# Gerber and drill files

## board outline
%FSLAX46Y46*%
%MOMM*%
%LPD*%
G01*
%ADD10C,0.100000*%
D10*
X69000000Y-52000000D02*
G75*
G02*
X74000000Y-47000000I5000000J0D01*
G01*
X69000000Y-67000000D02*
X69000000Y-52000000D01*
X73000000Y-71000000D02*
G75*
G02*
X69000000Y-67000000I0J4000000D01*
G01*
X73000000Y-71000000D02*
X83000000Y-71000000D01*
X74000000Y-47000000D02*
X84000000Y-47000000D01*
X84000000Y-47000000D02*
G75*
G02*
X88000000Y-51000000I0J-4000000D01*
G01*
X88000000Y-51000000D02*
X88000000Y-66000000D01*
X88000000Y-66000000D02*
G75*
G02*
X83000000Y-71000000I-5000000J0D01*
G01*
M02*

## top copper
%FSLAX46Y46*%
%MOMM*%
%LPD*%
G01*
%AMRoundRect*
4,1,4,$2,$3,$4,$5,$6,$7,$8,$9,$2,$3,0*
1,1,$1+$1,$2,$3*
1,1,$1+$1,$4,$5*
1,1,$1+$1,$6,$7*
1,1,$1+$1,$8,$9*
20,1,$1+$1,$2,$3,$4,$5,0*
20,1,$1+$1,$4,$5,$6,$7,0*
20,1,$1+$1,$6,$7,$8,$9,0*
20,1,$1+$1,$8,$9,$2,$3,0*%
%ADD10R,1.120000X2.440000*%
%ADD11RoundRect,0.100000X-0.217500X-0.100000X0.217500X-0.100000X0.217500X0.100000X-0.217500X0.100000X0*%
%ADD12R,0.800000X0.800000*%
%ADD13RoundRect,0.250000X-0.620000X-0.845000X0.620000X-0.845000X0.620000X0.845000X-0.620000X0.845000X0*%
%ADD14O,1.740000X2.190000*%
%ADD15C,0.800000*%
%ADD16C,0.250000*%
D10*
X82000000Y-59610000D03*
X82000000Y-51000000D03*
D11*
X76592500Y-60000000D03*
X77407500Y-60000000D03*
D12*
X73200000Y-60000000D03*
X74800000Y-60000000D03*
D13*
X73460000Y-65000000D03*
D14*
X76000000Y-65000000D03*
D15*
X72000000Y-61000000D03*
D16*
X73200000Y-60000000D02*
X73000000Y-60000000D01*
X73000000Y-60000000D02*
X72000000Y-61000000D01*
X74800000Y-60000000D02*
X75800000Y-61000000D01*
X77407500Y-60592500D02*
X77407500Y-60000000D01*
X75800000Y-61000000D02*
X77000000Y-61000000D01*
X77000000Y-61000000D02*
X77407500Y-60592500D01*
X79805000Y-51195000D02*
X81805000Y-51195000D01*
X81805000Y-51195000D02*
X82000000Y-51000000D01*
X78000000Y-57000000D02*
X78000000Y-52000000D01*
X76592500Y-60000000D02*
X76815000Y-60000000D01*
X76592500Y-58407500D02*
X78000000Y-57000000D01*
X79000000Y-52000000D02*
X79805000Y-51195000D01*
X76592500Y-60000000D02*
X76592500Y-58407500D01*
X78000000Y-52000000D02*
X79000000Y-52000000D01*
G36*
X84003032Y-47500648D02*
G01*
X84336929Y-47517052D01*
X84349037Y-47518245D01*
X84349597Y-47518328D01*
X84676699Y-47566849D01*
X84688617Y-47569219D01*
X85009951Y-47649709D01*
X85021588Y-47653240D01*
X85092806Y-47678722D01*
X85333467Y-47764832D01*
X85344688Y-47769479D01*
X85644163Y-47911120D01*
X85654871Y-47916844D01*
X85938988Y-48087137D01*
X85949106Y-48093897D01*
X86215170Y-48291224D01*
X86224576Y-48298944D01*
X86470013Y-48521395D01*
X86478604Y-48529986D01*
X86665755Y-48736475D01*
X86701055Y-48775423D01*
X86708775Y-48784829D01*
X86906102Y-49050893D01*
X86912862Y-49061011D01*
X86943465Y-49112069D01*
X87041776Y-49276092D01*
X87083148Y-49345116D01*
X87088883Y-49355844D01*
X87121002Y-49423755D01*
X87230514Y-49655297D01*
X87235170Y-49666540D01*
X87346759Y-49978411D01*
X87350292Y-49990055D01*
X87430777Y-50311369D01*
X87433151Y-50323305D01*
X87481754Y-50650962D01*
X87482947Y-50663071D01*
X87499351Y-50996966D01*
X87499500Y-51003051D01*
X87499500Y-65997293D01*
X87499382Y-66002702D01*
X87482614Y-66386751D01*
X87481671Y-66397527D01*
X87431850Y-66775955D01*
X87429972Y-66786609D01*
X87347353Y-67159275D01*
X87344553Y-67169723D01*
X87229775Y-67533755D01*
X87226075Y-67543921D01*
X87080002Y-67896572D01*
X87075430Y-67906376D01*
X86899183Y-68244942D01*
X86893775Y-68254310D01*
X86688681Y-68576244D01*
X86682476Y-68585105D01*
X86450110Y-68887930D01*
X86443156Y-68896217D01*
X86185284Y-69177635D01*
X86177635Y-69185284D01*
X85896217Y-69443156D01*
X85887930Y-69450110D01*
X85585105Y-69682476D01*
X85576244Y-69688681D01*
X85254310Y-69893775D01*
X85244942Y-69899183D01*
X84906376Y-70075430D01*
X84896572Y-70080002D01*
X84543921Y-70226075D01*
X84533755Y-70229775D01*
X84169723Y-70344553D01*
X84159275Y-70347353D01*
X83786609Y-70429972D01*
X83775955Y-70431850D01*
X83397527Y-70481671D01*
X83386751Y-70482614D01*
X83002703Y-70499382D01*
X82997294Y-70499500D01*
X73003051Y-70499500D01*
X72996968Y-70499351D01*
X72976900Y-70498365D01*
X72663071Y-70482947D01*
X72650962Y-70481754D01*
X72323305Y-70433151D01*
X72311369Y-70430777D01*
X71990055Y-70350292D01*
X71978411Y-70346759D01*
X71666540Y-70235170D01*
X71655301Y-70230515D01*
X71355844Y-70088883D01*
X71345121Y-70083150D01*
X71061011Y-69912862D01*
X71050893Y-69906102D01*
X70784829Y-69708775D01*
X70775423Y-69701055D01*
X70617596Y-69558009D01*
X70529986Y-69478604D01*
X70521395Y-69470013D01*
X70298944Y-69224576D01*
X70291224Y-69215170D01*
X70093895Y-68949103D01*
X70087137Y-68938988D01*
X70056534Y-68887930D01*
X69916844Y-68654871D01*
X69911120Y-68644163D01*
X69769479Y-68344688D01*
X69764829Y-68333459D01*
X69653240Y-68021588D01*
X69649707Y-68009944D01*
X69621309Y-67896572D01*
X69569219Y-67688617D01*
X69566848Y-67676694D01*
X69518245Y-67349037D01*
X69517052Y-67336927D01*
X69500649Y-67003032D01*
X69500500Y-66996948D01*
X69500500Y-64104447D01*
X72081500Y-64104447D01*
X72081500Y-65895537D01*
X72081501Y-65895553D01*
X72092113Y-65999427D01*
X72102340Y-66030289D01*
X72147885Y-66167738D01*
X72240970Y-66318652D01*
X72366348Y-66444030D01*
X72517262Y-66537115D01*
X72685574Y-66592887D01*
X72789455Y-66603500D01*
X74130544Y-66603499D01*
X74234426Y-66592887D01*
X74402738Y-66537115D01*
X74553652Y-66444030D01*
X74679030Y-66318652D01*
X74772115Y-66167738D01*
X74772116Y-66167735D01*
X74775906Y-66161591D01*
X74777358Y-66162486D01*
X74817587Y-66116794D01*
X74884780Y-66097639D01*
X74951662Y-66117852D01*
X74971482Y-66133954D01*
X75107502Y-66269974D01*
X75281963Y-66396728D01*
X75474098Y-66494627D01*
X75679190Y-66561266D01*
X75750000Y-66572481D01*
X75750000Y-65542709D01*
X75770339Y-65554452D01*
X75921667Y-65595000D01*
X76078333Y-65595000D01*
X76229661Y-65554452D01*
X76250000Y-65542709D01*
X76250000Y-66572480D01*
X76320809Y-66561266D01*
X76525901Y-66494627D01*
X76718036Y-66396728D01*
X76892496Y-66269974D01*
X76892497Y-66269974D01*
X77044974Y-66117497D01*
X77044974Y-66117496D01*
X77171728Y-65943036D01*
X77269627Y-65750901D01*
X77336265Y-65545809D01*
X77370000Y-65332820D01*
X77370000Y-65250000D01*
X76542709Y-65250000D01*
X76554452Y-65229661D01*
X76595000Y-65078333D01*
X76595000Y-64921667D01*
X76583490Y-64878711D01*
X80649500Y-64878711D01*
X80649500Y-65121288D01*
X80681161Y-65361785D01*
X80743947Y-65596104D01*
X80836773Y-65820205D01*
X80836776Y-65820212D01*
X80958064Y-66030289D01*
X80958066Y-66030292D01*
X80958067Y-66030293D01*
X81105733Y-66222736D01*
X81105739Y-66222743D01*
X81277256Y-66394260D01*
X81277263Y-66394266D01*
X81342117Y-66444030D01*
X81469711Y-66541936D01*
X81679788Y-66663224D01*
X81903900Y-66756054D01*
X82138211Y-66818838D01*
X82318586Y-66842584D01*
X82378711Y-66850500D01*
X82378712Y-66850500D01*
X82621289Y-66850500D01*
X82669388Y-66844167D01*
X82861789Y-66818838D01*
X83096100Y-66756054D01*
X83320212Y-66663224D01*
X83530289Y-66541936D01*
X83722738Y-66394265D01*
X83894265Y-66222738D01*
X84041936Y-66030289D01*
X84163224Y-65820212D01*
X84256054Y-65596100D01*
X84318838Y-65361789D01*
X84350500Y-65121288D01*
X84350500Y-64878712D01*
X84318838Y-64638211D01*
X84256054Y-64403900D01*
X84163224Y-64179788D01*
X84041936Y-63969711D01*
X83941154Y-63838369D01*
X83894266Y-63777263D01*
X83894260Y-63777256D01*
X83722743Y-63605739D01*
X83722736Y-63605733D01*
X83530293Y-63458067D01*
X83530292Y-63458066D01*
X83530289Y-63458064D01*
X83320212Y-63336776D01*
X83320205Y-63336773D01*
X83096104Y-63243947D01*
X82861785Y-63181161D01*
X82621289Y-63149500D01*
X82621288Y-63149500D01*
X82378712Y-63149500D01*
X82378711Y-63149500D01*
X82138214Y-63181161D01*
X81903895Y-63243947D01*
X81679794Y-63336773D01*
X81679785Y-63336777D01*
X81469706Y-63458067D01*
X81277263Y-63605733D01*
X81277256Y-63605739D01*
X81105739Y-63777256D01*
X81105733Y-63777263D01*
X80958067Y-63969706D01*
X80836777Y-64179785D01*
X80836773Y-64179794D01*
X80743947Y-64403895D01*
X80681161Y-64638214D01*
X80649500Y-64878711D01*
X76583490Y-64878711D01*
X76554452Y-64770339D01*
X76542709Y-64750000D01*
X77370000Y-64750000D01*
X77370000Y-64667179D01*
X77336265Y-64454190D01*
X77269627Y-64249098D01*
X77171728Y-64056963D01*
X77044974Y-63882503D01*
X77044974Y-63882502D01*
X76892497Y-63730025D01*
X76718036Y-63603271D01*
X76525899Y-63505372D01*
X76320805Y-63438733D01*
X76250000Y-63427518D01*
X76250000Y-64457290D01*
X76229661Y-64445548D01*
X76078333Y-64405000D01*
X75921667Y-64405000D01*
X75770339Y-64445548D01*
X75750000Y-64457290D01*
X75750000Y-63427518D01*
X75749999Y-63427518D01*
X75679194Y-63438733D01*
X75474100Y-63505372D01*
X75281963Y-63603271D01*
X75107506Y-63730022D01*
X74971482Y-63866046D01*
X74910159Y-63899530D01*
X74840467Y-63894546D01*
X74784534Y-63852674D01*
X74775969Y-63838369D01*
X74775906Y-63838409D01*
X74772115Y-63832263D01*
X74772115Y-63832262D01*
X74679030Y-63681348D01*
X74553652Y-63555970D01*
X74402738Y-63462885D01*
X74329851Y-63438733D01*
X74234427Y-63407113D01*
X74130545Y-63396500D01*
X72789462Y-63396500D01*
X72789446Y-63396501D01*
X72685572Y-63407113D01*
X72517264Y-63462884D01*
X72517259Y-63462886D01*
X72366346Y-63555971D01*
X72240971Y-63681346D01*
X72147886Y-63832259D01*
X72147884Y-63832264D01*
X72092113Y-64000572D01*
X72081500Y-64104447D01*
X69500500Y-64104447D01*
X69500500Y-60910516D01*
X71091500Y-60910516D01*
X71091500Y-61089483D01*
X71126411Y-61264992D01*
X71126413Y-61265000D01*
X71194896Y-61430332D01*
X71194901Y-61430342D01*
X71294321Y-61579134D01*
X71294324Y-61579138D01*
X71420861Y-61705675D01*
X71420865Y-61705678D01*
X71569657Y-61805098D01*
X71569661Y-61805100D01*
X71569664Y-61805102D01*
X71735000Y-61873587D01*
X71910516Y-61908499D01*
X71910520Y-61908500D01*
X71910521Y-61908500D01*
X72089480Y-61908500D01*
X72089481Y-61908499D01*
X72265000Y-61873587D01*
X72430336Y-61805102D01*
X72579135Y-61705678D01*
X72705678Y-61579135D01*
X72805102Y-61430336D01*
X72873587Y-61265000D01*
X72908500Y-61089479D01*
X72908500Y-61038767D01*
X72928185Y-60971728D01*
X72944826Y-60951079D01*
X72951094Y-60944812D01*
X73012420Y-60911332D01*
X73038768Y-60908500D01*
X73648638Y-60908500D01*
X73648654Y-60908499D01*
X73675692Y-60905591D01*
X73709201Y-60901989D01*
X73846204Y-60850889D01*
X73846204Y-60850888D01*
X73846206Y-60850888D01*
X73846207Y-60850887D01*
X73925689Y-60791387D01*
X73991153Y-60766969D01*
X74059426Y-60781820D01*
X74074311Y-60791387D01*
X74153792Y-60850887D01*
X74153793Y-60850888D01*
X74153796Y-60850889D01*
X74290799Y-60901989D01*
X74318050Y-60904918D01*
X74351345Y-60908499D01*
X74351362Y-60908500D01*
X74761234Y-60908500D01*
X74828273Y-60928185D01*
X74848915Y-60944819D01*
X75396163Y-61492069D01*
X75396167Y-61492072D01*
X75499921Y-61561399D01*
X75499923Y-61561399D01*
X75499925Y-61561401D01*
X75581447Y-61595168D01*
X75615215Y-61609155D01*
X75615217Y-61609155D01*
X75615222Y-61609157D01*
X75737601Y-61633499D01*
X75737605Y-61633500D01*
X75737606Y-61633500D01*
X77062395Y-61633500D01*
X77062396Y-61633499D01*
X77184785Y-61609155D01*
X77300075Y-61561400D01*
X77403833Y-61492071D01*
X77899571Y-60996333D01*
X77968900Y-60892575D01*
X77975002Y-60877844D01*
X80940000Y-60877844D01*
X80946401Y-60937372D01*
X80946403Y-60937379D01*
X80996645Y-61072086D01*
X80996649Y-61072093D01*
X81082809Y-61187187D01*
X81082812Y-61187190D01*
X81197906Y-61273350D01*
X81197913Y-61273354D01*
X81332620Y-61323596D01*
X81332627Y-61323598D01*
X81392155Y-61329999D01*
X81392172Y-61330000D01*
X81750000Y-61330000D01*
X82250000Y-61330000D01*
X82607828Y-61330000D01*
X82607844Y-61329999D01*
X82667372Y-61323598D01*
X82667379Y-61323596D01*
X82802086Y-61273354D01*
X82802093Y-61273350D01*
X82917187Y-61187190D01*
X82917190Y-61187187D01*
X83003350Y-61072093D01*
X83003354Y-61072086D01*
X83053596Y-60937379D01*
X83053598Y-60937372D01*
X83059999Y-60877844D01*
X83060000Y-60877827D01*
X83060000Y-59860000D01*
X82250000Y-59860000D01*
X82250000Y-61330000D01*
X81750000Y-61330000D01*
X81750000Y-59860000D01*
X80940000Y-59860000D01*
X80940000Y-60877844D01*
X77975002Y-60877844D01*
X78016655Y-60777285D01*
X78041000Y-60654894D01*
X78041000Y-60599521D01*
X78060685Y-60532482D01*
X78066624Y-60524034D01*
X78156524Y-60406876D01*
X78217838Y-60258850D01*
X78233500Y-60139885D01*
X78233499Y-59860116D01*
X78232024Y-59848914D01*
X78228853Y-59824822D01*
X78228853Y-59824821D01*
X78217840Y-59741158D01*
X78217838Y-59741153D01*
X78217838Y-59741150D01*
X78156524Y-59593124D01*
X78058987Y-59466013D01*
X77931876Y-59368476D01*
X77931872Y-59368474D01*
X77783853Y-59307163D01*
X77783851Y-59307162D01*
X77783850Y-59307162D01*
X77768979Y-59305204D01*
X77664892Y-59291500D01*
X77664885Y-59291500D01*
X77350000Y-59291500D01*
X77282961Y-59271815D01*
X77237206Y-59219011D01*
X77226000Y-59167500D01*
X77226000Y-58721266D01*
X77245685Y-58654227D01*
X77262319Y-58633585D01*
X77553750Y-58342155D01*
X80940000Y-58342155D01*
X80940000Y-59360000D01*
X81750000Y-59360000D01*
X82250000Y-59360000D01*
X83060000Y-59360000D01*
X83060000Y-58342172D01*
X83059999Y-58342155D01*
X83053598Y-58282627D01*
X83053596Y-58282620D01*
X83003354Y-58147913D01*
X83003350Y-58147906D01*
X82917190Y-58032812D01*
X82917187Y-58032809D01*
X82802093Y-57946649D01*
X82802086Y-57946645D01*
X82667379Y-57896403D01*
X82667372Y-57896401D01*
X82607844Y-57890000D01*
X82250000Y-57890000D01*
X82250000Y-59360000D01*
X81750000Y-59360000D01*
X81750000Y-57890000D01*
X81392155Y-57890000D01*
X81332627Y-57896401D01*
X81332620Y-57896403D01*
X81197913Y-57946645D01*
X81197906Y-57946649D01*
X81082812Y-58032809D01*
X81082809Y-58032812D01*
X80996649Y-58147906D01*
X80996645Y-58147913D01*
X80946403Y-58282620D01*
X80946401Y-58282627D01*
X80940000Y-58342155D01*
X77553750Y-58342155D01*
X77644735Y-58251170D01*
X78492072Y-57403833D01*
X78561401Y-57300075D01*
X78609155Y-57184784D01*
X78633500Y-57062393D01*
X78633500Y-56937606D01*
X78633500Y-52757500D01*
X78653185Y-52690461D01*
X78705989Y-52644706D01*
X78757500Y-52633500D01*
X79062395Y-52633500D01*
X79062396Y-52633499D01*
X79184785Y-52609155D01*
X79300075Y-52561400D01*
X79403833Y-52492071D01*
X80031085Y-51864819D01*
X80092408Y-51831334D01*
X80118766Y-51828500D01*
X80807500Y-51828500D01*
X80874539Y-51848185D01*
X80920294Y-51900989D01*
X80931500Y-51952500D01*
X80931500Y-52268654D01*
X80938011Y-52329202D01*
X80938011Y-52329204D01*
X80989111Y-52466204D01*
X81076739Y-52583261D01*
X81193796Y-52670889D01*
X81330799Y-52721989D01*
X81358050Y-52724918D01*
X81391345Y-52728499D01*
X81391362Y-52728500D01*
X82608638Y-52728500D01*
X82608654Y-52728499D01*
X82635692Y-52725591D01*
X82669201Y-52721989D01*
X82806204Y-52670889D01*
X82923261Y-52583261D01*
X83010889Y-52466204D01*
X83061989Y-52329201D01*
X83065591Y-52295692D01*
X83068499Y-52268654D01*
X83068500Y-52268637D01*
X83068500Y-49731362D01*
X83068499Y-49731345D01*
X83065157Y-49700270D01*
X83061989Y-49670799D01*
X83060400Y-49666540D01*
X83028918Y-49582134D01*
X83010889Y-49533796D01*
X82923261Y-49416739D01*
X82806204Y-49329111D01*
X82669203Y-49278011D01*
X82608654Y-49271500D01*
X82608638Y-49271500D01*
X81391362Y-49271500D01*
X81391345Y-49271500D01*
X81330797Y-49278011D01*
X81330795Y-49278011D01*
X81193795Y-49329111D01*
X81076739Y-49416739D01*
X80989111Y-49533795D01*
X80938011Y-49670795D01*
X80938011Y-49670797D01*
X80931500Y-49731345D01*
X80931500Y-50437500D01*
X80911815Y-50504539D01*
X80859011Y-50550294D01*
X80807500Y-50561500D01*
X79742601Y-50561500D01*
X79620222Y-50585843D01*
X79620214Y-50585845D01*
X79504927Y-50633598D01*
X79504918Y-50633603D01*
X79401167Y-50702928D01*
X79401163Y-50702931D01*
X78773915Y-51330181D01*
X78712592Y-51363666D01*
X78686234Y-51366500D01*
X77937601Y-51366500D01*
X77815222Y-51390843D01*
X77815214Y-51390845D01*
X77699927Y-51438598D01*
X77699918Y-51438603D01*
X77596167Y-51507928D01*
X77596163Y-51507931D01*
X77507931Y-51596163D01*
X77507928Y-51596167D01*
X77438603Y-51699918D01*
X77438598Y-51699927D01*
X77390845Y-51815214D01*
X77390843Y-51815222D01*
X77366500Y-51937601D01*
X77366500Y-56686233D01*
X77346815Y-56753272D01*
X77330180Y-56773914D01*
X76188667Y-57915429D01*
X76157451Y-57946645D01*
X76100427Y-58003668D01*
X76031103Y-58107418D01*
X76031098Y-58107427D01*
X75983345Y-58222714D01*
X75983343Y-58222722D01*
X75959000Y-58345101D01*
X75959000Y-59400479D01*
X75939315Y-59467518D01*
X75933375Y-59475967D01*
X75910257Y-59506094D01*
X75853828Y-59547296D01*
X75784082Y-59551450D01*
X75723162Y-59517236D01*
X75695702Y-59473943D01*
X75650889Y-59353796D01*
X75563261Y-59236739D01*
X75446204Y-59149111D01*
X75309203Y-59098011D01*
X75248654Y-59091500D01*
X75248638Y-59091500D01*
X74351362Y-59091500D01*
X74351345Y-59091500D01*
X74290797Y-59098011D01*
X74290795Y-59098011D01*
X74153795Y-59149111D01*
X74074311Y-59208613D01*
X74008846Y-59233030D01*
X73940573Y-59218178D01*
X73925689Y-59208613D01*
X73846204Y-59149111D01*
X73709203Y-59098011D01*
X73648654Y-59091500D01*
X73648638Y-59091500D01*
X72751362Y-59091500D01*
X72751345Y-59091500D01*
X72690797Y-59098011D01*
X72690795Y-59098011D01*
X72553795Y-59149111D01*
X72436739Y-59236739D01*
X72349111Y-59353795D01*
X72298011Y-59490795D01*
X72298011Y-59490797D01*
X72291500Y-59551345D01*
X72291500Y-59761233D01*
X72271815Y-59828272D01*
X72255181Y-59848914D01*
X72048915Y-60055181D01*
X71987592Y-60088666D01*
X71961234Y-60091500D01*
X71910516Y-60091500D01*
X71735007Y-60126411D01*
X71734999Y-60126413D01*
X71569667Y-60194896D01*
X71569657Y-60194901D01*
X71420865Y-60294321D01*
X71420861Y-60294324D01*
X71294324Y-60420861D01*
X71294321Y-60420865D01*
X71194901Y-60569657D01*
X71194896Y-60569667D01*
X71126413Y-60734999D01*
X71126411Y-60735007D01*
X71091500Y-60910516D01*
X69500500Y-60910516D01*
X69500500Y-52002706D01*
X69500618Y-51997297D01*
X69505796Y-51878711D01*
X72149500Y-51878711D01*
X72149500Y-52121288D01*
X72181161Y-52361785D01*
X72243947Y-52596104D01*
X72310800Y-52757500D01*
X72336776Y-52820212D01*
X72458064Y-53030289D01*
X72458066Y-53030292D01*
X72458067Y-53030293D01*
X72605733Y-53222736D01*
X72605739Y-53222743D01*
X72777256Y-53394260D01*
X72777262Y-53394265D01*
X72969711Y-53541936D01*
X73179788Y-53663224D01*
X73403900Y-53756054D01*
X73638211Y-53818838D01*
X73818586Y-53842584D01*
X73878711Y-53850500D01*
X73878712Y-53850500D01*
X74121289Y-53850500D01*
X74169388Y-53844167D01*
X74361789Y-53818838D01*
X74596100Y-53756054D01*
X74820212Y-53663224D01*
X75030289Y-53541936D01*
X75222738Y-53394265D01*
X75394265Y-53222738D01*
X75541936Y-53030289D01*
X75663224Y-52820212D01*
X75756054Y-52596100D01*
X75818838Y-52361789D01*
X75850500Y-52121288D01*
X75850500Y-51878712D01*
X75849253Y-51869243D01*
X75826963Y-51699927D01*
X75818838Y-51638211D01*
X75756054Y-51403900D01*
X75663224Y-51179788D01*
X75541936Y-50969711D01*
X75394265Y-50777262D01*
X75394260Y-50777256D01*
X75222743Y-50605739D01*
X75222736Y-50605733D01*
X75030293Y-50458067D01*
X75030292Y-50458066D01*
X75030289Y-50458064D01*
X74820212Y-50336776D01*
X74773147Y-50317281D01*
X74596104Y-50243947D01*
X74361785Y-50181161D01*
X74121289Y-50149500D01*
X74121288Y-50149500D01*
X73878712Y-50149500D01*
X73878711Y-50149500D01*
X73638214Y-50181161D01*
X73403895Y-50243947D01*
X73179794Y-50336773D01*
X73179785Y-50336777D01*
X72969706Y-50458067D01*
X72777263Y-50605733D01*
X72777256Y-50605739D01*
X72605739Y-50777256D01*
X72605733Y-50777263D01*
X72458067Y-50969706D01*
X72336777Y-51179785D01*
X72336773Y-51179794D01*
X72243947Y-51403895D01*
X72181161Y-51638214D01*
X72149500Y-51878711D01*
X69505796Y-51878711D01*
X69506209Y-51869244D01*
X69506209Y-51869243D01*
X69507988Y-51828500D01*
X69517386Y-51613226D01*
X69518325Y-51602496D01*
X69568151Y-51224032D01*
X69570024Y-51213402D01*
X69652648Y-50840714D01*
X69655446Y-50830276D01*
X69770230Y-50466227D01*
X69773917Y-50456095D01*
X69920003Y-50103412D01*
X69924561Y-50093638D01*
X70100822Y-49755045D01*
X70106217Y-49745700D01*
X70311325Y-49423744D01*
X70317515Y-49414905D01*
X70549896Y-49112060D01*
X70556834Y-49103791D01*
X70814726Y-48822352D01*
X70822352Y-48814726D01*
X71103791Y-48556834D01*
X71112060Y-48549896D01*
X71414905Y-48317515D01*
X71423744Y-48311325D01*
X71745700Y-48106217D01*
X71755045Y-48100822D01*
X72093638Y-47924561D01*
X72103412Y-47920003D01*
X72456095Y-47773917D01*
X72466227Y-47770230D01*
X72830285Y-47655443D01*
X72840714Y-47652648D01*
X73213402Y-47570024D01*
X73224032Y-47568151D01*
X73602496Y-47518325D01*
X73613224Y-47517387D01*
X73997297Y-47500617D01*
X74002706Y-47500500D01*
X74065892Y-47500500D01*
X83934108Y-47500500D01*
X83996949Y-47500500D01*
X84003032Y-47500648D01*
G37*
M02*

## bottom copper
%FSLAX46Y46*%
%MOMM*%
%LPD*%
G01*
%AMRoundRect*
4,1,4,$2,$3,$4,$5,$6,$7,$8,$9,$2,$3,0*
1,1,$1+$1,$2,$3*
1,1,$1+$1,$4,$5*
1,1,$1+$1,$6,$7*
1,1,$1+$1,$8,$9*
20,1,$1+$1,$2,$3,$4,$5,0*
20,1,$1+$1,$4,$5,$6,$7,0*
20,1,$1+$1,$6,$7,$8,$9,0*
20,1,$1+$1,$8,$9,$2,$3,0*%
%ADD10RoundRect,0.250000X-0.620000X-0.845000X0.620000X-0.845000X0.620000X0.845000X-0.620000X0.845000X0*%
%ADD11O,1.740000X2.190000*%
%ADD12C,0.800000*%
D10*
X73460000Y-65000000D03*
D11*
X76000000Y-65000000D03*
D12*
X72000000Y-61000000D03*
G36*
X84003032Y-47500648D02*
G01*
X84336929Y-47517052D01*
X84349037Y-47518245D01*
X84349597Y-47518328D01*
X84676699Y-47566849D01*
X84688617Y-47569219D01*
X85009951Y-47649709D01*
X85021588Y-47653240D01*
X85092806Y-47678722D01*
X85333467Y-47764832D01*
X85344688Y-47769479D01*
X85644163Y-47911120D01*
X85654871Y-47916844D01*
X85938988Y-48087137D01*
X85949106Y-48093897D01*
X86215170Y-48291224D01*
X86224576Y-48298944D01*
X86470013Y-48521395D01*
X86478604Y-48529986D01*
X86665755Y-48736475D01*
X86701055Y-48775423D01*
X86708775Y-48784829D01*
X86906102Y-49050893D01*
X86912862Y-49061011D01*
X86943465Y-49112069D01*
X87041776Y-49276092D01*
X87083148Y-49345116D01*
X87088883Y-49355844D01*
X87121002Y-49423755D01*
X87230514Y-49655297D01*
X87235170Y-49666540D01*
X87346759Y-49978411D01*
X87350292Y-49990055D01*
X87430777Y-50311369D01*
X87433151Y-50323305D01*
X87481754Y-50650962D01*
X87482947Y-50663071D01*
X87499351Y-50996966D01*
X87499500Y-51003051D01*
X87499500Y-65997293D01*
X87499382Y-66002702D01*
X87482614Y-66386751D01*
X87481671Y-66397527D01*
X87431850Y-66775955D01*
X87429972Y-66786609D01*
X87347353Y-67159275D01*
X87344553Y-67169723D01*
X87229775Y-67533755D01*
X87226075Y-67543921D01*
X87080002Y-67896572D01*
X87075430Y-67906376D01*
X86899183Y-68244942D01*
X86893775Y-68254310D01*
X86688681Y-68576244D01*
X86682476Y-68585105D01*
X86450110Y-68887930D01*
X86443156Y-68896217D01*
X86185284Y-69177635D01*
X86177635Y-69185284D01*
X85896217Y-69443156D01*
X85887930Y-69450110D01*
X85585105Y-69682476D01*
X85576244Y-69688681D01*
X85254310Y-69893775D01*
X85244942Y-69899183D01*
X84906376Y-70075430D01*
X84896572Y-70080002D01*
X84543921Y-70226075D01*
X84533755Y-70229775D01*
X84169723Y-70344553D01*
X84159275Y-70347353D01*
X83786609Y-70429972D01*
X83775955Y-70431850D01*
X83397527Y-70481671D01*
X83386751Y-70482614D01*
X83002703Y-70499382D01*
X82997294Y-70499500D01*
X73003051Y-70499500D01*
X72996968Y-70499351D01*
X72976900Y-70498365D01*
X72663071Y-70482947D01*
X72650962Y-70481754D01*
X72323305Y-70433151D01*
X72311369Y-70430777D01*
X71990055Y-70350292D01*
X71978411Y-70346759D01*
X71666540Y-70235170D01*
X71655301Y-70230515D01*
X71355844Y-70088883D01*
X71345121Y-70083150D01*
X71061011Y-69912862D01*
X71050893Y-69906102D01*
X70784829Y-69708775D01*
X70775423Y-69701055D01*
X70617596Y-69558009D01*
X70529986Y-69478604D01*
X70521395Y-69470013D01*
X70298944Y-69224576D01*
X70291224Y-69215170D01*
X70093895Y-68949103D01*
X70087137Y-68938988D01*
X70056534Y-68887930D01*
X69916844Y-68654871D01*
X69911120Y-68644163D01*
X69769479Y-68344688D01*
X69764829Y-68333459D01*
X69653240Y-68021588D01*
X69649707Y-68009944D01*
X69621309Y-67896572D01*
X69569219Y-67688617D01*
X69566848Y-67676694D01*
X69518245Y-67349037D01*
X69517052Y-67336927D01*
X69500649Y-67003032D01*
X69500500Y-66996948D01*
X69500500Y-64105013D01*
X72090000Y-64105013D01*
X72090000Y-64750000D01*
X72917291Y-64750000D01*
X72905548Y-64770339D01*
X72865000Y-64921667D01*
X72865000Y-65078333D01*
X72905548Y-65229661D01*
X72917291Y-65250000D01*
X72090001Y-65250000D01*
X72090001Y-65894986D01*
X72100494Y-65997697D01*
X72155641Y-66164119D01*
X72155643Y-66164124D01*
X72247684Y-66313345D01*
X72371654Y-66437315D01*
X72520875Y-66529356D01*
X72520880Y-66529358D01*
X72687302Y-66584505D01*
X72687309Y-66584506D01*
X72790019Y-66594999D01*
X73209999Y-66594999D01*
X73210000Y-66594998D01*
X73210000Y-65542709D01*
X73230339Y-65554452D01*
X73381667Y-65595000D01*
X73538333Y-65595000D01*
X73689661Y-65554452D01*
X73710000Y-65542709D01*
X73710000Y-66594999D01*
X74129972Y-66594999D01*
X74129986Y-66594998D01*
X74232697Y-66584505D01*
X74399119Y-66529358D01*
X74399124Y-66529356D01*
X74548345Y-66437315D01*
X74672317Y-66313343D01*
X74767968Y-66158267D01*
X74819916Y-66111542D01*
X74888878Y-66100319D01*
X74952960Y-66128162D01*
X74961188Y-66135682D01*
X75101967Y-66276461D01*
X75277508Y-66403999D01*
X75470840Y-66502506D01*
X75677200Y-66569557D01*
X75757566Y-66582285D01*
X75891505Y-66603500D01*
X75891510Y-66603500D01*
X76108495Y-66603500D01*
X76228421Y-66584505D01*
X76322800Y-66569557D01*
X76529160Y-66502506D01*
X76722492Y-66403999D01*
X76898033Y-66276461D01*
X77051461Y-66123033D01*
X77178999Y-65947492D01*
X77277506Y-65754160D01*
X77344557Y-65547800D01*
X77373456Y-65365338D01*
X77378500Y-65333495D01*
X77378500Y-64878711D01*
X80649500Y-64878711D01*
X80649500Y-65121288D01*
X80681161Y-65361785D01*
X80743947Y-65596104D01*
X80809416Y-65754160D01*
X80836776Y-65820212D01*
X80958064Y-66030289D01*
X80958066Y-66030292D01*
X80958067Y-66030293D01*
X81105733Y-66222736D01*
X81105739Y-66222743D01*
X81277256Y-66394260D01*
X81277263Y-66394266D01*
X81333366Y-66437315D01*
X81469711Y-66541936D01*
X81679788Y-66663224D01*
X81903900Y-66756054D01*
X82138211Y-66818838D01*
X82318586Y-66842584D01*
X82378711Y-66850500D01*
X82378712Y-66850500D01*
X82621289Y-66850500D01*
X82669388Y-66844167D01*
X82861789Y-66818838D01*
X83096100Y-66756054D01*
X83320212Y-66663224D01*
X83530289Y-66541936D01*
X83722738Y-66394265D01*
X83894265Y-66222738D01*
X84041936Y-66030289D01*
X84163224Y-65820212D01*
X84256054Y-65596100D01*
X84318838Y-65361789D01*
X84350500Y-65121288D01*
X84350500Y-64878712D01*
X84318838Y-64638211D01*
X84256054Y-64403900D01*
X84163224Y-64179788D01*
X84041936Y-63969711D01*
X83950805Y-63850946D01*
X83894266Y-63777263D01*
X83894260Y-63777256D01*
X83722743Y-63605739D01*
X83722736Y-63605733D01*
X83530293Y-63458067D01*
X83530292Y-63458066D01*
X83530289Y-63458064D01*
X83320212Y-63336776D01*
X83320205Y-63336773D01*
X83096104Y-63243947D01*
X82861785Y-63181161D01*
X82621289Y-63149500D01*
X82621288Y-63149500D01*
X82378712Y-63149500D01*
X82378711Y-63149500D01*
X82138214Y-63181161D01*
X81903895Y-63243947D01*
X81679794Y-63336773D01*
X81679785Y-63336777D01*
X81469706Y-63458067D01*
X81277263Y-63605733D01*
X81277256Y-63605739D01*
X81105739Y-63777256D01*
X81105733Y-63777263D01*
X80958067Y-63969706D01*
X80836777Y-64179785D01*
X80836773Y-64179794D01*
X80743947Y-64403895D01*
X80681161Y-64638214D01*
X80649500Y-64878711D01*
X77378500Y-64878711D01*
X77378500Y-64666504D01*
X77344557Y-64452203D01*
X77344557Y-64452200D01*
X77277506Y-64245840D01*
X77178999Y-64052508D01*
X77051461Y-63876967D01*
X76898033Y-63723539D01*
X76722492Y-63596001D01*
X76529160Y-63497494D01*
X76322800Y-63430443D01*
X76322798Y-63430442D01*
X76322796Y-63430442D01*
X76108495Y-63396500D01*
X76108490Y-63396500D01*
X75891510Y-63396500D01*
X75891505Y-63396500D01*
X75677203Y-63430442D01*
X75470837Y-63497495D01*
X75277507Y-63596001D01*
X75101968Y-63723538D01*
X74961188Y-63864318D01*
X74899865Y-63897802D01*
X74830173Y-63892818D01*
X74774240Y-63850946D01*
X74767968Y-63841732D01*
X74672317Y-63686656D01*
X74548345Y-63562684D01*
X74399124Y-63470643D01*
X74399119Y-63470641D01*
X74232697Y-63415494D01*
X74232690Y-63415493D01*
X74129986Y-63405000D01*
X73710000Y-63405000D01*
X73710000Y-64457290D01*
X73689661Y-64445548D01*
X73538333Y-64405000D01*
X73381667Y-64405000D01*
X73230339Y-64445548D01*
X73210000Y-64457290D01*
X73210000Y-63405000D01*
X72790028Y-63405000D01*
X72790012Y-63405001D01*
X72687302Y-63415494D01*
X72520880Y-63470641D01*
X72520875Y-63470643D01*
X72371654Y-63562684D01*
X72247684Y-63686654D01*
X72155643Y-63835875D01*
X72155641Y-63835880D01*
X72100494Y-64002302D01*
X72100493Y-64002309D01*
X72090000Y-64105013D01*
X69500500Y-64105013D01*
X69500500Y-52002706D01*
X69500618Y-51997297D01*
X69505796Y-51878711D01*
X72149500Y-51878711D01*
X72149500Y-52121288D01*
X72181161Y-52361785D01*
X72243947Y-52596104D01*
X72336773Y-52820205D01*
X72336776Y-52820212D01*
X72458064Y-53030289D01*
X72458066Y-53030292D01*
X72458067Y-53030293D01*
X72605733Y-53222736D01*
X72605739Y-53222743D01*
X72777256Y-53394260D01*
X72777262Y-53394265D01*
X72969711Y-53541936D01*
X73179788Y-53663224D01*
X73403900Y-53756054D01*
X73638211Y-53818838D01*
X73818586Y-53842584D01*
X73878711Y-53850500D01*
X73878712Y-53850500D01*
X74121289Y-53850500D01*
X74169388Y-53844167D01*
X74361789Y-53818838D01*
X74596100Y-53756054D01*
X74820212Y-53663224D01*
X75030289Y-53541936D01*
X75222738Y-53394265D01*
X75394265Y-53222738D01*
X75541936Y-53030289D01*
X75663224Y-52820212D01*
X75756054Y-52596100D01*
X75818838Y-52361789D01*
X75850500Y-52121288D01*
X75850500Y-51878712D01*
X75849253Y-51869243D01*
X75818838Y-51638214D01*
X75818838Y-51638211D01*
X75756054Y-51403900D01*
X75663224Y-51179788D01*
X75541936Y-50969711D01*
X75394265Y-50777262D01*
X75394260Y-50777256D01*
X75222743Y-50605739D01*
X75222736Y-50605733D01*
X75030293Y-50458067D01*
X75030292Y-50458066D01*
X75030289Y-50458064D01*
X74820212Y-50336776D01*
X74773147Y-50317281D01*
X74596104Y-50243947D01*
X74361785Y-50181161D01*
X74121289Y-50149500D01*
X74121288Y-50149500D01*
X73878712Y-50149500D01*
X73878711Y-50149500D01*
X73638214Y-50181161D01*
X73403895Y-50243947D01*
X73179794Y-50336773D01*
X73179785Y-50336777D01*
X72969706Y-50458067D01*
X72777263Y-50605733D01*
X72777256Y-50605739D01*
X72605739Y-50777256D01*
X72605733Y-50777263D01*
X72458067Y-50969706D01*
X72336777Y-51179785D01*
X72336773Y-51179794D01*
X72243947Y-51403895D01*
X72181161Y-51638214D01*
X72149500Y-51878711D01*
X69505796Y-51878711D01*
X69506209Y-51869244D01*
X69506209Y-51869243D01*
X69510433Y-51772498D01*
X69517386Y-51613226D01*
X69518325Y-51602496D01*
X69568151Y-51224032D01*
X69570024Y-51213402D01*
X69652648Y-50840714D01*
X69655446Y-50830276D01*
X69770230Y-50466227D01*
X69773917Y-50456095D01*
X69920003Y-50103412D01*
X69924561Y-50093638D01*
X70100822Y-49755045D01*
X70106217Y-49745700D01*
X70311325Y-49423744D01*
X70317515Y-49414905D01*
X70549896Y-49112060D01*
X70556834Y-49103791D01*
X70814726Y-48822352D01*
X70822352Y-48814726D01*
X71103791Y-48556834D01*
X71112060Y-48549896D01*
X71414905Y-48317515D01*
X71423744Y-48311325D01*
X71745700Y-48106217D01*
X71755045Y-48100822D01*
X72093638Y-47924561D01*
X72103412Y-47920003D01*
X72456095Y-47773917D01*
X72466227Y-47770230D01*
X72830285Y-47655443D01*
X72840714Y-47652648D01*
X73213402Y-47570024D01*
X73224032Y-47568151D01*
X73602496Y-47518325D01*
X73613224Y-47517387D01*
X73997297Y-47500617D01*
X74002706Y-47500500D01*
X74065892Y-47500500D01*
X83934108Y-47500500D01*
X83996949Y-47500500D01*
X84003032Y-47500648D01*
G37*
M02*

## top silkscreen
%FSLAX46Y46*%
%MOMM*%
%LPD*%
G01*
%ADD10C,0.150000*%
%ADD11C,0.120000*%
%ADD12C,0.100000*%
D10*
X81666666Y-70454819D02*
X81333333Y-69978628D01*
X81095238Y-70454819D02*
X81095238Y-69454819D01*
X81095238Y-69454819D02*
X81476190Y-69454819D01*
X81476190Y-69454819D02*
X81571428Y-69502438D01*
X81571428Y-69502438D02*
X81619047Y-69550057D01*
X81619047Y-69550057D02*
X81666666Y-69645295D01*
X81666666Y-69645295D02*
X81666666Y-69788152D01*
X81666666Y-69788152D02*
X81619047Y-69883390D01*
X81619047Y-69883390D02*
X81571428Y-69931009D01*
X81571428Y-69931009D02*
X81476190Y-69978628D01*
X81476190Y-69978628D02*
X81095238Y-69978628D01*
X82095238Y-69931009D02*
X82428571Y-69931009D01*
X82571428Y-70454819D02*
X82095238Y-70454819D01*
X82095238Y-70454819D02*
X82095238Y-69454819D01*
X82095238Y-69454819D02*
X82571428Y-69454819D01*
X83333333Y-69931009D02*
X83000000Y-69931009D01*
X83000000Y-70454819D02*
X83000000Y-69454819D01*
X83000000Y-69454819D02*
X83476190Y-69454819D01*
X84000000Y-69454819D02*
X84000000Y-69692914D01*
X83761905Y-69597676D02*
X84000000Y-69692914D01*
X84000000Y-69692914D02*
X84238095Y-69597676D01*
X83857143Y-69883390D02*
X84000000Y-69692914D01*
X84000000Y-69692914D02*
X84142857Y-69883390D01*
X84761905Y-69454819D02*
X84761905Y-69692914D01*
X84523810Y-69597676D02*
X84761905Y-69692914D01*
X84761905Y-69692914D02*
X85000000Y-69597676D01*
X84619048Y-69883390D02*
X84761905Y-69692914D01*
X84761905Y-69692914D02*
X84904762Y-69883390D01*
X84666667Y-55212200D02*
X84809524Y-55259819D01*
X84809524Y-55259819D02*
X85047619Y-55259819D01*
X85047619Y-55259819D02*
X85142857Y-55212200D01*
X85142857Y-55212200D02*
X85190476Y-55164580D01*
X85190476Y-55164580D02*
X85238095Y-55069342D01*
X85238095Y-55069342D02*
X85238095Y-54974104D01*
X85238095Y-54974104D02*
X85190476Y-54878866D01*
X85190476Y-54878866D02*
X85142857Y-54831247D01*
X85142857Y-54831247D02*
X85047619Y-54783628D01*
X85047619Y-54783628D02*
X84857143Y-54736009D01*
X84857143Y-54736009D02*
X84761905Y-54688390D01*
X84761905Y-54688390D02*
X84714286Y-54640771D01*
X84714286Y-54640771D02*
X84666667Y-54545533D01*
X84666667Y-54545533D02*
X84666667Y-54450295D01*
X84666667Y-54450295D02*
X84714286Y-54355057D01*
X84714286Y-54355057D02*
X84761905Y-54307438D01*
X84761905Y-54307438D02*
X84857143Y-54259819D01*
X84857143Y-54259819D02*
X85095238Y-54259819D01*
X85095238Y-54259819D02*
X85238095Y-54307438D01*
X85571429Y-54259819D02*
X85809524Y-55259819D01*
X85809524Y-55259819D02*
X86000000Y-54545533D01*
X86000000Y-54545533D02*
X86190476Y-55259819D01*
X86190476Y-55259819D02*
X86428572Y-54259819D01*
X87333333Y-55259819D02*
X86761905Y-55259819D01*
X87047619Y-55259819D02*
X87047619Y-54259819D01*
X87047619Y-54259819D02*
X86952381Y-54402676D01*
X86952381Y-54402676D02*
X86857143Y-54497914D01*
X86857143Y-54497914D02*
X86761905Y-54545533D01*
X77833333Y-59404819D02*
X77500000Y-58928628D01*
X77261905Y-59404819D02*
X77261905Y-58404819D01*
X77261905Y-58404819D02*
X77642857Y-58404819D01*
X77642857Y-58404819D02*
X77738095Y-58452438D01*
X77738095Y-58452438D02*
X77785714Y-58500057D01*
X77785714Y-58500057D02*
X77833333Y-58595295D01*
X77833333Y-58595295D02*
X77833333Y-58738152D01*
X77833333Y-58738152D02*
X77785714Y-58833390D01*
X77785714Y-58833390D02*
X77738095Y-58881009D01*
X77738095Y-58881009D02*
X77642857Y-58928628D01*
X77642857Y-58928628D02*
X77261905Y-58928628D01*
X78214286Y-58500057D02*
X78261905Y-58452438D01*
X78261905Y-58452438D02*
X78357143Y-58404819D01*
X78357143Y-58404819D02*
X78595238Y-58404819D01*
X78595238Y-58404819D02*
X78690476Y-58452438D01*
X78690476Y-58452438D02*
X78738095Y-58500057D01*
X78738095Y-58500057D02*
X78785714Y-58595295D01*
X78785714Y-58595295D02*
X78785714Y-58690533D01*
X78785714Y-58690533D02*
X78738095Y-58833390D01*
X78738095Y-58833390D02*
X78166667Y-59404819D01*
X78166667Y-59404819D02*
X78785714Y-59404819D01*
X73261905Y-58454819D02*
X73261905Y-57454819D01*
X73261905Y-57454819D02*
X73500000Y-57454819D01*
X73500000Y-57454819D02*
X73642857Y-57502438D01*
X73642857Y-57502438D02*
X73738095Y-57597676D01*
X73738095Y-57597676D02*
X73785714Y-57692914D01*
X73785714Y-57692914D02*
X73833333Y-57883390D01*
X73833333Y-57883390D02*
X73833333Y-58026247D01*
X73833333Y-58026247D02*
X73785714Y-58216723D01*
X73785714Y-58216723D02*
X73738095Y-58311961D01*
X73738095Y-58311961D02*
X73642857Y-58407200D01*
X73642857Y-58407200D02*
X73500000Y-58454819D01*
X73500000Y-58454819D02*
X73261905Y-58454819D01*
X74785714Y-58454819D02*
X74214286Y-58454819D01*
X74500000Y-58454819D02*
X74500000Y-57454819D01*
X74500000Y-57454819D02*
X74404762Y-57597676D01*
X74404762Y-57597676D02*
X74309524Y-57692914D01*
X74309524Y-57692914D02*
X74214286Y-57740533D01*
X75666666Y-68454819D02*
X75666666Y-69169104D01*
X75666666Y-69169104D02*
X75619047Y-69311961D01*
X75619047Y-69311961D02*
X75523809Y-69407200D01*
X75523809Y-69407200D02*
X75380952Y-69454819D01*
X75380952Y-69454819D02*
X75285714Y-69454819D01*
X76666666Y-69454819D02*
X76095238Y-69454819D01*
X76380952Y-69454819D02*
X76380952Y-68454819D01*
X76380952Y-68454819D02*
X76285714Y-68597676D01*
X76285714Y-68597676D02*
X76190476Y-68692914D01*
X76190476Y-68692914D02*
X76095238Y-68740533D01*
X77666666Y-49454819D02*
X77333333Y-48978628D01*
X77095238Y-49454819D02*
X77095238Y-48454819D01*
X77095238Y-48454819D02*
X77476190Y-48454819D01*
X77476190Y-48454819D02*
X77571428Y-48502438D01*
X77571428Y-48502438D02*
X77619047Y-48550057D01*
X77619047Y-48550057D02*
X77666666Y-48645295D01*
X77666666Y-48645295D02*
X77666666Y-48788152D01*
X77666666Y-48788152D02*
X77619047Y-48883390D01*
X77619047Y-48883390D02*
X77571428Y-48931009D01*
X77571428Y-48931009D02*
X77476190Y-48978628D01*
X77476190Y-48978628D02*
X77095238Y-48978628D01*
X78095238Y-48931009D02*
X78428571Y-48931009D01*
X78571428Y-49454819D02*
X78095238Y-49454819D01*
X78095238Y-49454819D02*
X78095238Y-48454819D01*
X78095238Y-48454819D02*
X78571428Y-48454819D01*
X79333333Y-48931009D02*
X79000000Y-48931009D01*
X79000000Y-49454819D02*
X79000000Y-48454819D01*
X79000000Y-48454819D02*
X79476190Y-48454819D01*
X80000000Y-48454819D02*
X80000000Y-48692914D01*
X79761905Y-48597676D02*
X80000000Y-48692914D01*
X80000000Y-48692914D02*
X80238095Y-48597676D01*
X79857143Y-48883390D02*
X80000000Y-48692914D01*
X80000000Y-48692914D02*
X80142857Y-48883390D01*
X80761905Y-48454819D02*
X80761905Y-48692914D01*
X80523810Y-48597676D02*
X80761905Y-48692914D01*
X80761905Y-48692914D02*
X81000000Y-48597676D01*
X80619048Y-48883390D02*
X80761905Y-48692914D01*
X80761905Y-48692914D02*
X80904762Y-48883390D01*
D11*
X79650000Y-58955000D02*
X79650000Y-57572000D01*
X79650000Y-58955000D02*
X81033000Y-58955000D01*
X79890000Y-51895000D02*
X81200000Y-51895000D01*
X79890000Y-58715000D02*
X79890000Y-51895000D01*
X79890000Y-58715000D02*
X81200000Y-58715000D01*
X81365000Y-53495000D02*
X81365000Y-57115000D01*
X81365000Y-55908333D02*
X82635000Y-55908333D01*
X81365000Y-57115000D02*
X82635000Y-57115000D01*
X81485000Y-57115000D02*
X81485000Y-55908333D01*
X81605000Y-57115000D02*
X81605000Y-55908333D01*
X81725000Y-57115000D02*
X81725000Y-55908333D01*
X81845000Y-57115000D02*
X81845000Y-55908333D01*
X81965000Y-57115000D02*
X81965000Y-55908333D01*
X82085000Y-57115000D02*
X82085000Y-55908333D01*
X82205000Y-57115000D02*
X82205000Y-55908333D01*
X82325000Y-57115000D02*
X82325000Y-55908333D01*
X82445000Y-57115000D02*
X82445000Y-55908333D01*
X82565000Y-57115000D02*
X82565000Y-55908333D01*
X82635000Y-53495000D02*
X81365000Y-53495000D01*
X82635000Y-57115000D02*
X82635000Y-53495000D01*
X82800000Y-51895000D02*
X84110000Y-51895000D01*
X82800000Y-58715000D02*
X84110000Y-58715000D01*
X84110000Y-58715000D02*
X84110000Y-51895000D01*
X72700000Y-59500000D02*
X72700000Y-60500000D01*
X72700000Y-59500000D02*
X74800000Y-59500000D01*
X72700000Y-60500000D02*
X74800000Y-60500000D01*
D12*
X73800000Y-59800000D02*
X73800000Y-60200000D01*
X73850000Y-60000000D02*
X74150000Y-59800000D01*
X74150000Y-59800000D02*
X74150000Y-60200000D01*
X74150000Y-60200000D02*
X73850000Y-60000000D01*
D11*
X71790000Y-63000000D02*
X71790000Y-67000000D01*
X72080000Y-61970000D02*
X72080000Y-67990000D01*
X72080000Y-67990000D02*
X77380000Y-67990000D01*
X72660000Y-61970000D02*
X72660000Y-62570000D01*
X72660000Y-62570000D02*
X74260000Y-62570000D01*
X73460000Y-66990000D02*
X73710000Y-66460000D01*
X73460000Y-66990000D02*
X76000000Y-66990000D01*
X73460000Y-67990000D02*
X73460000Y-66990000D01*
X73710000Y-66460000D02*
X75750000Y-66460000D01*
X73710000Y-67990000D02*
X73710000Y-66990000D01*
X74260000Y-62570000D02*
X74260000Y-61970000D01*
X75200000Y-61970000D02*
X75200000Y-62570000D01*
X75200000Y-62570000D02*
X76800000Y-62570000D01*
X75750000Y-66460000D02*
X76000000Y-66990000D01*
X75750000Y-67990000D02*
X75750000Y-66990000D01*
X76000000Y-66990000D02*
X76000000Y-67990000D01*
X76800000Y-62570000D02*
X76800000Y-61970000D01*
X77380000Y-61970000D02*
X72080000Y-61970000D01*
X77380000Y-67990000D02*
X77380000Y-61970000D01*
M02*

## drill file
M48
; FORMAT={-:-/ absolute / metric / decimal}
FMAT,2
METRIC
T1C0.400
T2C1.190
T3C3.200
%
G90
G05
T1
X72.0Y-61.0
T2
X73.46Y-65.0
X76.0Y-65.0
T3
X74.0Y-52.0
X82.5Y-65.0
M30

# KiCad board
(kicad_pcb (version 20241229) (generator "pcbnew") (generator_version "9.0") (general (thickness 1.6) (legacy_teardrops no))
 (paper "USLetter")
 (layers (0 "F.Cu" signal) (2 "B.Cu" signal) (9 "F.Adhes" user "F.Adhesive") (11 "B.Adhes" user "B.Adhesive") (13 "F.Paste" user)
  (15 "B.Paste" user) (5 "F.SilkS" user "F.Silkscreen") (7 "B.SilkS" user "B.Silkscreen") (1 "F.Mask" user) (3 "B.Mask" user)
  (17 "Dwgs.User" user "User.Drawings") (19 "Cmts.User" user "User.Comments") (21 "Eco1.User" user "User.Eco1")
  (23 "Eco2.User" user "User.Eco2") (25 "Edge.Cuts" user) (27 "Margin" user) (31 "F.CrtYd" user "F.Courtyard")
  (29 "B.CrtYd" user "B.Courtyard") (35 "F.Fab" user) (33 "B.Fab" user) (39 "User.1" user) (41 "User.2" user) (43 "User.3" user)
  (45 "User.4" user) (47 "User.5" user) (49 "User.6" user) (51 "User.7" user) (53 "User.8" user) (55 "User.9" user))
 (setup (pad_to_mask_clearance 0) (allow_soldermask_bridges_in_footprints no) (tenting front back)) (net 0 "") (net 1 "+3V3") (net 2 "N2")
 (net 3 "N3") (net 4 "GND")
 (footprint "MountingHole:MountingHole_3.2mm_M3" (layer "F.Cu") (at 82.5 65)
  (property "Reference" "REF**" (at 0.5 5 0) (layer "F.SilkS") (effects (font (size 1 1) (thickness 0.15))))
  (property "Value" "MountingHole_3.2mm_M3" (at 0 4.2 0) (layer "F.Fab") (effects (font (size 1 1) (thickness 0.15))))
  (pad "" np_thru_hole circle (at 0 0) (size 3.2 3.2) (drill 3.2) (layers "*.Cu" "*.Mask")))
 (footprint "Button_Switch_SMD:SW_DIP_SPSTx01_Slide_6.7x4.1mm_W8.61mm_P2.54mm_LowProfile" (layer "F.Cu") (at 82 55.305 90)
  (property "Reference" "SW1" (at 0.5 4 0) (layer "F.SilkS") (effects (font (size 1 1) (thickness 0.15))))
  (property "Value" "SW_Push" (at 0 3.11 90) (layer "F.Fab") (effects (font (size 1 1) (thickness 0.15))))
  (fp_line (start -3.65 -2.35) (end -2.267 -2.35) (stroke (width 0.12) (type solid)) (layer "F.SilkS"))
  (fp_line (start -3.65 -2.35) (end -3.65 -0.967) (stroke (width 0.12) (type solid)) (layer "F.SilkS"))
  (fp_line (start 3.41 -2.11) (end 3.41 -0.8) (stroke (width 0.12) (type solid)) (layer "F.SilkS"))
  (fp_line (start -3.41 -2.11) (end 3.41 -2.11) (stroke (width 0.12) (type solid)) (layer "F.SilkS"))
  (fp_line (start -3.41 -2.11) (end -3.41 -0.8) (stroke (width 0.12) (type solid)) (layer "F.SilkS"))
  (fp_line (start 1.81 -0.635) (end -1.81 -0.635) (stroke (width 0.12) (type solid)) (layer "F.SilkS"))
  (fp_line (start -0.603333 -0.635) (end -0.603333 0.635) (stroke (width 0.12) (type solid)) (layer "F.SilkS"))
  (fp_line (start -1.81 -0.635) (end -1.81 0.635) (stroke (width 0.12) (type solid)) (layer "F.SilkS"))
  (fp_line (start -1.81 -0.515) (end -0.603333 -0.515) (stroke (width 0.12) (type solid)) (layer "F.SilkS"))
  (fp_line (start -1.81 -0.395) (end -0.603333 -0.395) (stroke (width 0.12) (type solid)) (layer "F.SilkS"))
  (fp_line (start -1.81 -0.275) (end -0.603333 -0.275) (stroke (width 0.12) (type solid)) (layer "F.SilkS"))
  (fp_line (start -1.81 -0.155) (end -0.603333 -0.155) (stroke (width 0.12) (type solid)) (layer "F.SilkS"))
  (fp_line (start -1.81 -0.035) (end -0.603333 -0.035) (stroke (width 0.12) (type solid)) (layer "F.SilkS"))
  (fp_line (start -1.81 0.085) (end -0.603333 0.085) (stroke (width 0.12) (type solid)) (layer "F.SilkS"))
  (fp_line (start -1.81 0.205) (end -0.603333 0.205) (stroke (width 0.12) (type solid)) (layer "F.SilkS"))
  (fp_line (start -1.81 0.325) (end -0.603333 0.325) (stroke (width 0.12) (type solid)) (layer "F.SilkS"))
  (fp_line (start -1.81 0.445) (end -0.603333 0.445) (stroke (width 0.12) (type solid)) (layer "F.SilkS"))
  (fp_line (start -1.81 0.565) (end -0.603333 0.565) (stroke (width 0.12) (type solid)) (layer "F.SilkS"))
  (fp_line (start 1.81 0.635) (end 1.81 -0.635) (stroke (width 0.12) (type solid)) (layer "F.SilkS"))
  (fp_line (start -1.81 0.635) (end 1.81 0.635) (stroke (width 0.12) (type solid)) (layer "F.SilkS"))
  (fp_line (start 3.41 0.8) (end 3.41 2.11) (stroke (width 0.12) (type solid)) (layer "F.SilkS"))
  (fp_line (start -3.41 0.8) (end -3.41 2.11) (stroke (width 0.12) (type solid)) (layer "F.SilkS"))
  (fp_line (start -3.41 2.11) (end 3.41 2.11) (stroke (width 0.12) (type solid)) (layer "F.SilkS"))
  (pad "1" smd rect (at -4.305 0 90) (size 2.44 1.12) (layers "F.Cu" "F.Mask" "F.Paste") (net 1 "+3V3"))
  (pad "2" smd rect (at 4.305 0 90) (size 2.44 1.12) (layers "F.Cu" "F.Mask" "F.Paste") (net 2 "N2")))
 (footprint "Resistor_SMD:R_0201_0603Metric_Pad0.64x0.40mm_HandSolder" (layer "F.Cu") (at 77 60)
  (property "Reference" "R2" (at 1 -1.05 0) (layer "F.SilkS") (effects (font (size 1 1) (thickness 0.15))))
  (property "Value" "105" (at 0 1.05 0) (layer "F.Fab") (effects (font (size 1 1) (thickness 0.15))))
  (pad "" smd roundrect (at -0.4325 0) (size 0.458 0.36) (layers "F.Paste") (roundrect_rratio 0.25))
  (pad "" smd roundrect (at 0.4325 0) (size 0.458 0.36) (layers "F.Paste") (roundrect_rratio 0.25))
  (pad "1" smd roundrect (at -0.4075 0) (size 0.635 0.4) (layers "F.Cu" "F.Mask") (roundrect_rratio 0.25) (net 2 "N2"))
  (pad "2" smd roundrect (at 0.4075 0) (size 0.635 0.4) (layers "F.Cu" "F.Mask") (roundrect_rratio 0.25) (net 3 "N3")))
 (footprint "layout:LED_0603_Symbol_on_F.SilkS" (layer "F.Cu") (at 74 60)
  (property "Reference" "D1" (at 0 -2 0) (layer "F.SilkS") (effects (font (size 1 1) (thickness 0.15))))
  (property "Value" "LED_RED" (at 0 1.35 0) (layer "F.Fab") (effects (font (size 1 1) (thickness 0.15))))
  (fp_line (start -1.3 -0.5) (end -1.3 0.5) (stroke (width 0.12) (type solid)) (layer "F.SilkS"))
  (fp_line (start -1.3 -0.5) (end 0.8 -0.5) (stroke (width 0.12) (type solid)) (layer "F.SilkS"))
  (fp_line (start -1.3 0.5) (end 0.8 0.5) (stroke (width 0.12) (type solid)) (layer "F.SilkS"))
  (fp_line (start -0.2 -0.2) (end -0.2 0.2) (stroke (width 0.1) (type solid)) (layer "F.SilkS"))
  (fp_line (start -0.15 0) (end 0.15 -0.2) (stroke (width 0.1) (type solid)) (layer "F.SilkS"))
  (fp_line (start 0.15 -0.2) (end 0.15 0.2) (stroke (width 0.1) (type solid)) (layer "F.SilkS"))
  (fp_line (start 0.15 0.2) (end -0.15 0) (stroke (width 0.1) (type solid)) (layer "F.SilkS"))
  (pad "1" smd rect (at -0.8 0 180) (size 0.8 0.8) (layers "F.Cu" "F.Mask" "F.Paste") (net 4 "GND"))
  (pad "2" smd rect (at 0.8 0 180) (size 0.8 0.8) (layers "F.Cu" "F.Mask" "F.Paste") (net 3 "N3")))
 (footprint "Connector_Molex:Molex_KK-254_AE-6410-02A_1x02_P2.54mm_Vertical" (layer "F.Cu") (at 73.46 65)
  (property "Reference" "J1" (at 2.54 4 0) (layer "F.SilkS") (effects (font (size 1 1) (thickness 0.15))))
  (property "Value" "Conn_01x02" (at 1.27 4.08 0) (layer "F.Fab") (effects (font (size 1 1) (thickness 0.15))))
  (fp_line (start -1.67 -2) (end -1.67 2) (stroke (width 0.12) (type solid)) (layer "F.SilkS"))
  (fp_line (start -1.38 -3.03) (end -1.38 2.99) (stroke (width 0.12) (type solid)) (layer "F.SilkS"))
  (fp_line (start -1.38 2.99) (end 3.92 2.99) (stroke (width 0.12) (type solid)) (layer "F.SilkS"))
  (fp_line (start -0.8 -3.03) (end -0.8 -2.43) (stroke (width 0.12) (type solid)) (layer "F.SilkS"))
  (fp_line (start -0.8 -2.43) (end 0.8 -2.43) (stroke (width 0.12) (type solid)) (layer "F.SilkS"))
  (fp_line (start 0 1.99) (end 0.25 1.46) (stroke (width 0.12) (type solid)) (layer "F.SilkS"))
  (fp_line (start 0 1.99) (end 2.54 1.99) (stroke (width 0.12) (type solid)) (layer "F.SilkS"))
  (fp_line (start 0 2.99) (end 0 1.99) (stroke (width 0.12) (type solid)) (layer "F.SilkS"))
  (fp_line (start 0.25 1.46) (end 2.29 1.46) (stroke (width 0.12) (type solid)) (layer "F.SilkS"))
  (fp_line (start 0.25 2.99) (end 0.25 1.99) (stroke (width 0.12) (type solid)) (layer "F.SilkS"))
  (fp_line (start 0.8 -2.43) (end 0.8 -3.03) (stroke (width 0.12) (type solid)) (layer "F.SilkS"))
  (fp_line (start 1.74 -3.03) (end 1.74 -2.43) (stroke (width 0.12) (type solid)) (layer "F.SilkS"))
  (fp_line (start 1.74 -2.43) (end 3.34 -2.43) (stroke (width 0.12) (type solid)) (layer "F.SilkS"))
  (fp_line (start 2.29 1.46) (end 2.54 1.99) (stroke (width 0.12) (type solid)) (layer "F.SilkS"))
  (fp_line (start 2.29 2.99) (end 2.29 1.99) (stroke (width 0.12) (type solid)) (layer "F.SilkS"))
  (fp_line (start 2.54 1.99) (end 2.54 2.99) (stroke (width 0.12) (type solid)) (layer "F.SilkS"))
  (fp_line (start 3.34 -2.43) (end 3.34 -3.03) (stroke (width 0.12) (type solid)) (layer "F.SilkS"))
  (fp_line (start 3.92 -3.03) (end -1.38 -3.03) (stroke (width 0.12) (type solid)) (layer "F.SilkS"))
  (fp_line (start 3.92 2.99) (end 3.92 -3.03) (stroke (width 0.12) (type solid)) (layer "F.SilkS"))
  (pad "1" thru_hole roundrect (at 0 0) (size 1.74 2.19) (drill 1.19) (layers "*.Cu" "*.Mask") (remove_unused_layers no)
   (roundrect_rratio 0.143678) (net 4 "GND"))
  (pad "2" thru_hole oval (at 2.54 0) (size 1.74 2.19) (drill 1.19) (layers "*.Cu" "*.Mask") (remove_unused_layers no) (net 1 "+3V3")))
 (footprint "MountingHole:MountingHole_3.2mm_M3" (layer "F.Cu") (at 74 52)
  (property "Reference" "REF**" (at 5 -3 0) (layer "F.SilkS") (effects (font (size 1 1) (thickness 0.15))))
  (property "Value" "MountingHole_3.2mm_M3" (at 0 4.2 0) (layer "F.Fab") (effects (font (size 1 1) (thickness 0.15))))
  (pad "" np_thru_hole circle (at 0 0) (size 3.2 3.2) (drill 3.2) (layers "*.Cu" "*.Mask")))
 (gr_arc (start 69 52) (mid 70.464466 48.464466) (end 74 47) (stroke (width 0.1) (type default)) (layer "Edge.Cuts"))
 (gr_line (start 69 67) (end 69 52) (stroke (width 0.1) (type default)) (layer "Edge.Cuts"))
 (gr_arc (start 73 71) (mid 70.171573 69.828427) (end 69 67) (stroke (width 0.1) (type default)) (layer "Edge.Cuts"))
 (gr_line (start 73 71) (end 83 71) (stroke (width 0.1) (type default)) (layer "Edge.Cuts"))
 (gr_line (start 74 47) (end 84 47) (stroke (width 0.1) (type default)) (layer "Edge.Cuts"))
 (gr_arc (start 84 47) (mid 86.828427 48.171573) (end 88 51) (stroke (width 0.1) (type default)) (layer "Edge.Cuts"))
 (gr_line (start 88 51) (end 88 66) (stroke (width 0.1) (type default)) (layer "Edge.Cuts"))
 (gr_arc (start 88 66) (mid 86.535534 69.535534) (end 83 71) (stroke (width 0.1) (type default)) (layer "Edge.Cuts"))
 (segment (start 73.2 60) (end 73 60) (width 0.25) (layer "F.Cu") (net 4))
 (segment (start 73 60) (end 72 61) (width 0.25) (layer "F.Cu") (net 4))
 (via (at 72 61) (size 0.8) (drill 0.4) (layers "F.Cu" "B.Cu") (free yes) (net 4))
 (segment (start 74.8 60) (end 75.8 61) (width 0.25) (layer "F.Cu") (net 3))
 (segment (start 77.4075 60.5925) (end 77.4075 60) (width 0.25) (layer "F.Cu") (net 3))
 (segment (start 75.8 61) (end 77 61) (width 0.25) (layer "F.Cu") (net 3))
 (segment (start 77 61) (end 77.4075 60.5925) (width 0.25) (layer "F.Cu") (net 3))
 (segment (start 79.805 51.195) (end 81.805 51.195) (width 0.25) (layer "F.Cu") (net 2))
 (segment (start 81.805 51.195) (end 82 51) (width 0.25) (layer "F.Cu") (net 2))
 (segment (start 78 57) (end 78 52) (width 0.25) (layer "F.Cu") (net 2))
 (segment (start 76.5925 60) (end 76.815 60) (width 0.25) (layer "F.Cu") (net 2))
 (segment (start 76.5925 58.4075) (end 78 57) (width 0.25) (layer "F.Cu") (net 2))
 (segment (start 79 52) (end 79.805 51.195) (width 0.25) (layer "F.Cu") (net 2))
 (segment (start 76.5925 60) (end 76.5925 58.4075) (width 0.25) (layer "F.Cu") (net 2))
 (segment (start 78 52) (end 79 52) (width 0.25) (layer "F.Cu") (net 2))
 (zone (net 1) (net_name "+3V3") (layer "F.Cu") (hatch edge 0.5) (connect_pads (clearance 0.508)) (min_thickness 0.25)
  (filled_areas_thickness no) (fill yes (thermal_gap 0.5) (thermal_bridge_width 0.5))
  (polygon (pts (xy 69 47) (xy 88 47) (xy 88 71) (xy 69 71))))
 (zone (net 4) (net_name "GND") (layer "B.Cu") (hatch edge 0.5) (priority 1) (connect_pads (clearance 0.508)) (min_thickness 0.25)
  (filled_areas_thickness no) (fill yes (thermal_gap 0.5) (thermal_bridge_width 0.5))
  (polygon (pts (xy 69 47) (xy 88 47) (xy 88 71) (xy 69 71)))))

